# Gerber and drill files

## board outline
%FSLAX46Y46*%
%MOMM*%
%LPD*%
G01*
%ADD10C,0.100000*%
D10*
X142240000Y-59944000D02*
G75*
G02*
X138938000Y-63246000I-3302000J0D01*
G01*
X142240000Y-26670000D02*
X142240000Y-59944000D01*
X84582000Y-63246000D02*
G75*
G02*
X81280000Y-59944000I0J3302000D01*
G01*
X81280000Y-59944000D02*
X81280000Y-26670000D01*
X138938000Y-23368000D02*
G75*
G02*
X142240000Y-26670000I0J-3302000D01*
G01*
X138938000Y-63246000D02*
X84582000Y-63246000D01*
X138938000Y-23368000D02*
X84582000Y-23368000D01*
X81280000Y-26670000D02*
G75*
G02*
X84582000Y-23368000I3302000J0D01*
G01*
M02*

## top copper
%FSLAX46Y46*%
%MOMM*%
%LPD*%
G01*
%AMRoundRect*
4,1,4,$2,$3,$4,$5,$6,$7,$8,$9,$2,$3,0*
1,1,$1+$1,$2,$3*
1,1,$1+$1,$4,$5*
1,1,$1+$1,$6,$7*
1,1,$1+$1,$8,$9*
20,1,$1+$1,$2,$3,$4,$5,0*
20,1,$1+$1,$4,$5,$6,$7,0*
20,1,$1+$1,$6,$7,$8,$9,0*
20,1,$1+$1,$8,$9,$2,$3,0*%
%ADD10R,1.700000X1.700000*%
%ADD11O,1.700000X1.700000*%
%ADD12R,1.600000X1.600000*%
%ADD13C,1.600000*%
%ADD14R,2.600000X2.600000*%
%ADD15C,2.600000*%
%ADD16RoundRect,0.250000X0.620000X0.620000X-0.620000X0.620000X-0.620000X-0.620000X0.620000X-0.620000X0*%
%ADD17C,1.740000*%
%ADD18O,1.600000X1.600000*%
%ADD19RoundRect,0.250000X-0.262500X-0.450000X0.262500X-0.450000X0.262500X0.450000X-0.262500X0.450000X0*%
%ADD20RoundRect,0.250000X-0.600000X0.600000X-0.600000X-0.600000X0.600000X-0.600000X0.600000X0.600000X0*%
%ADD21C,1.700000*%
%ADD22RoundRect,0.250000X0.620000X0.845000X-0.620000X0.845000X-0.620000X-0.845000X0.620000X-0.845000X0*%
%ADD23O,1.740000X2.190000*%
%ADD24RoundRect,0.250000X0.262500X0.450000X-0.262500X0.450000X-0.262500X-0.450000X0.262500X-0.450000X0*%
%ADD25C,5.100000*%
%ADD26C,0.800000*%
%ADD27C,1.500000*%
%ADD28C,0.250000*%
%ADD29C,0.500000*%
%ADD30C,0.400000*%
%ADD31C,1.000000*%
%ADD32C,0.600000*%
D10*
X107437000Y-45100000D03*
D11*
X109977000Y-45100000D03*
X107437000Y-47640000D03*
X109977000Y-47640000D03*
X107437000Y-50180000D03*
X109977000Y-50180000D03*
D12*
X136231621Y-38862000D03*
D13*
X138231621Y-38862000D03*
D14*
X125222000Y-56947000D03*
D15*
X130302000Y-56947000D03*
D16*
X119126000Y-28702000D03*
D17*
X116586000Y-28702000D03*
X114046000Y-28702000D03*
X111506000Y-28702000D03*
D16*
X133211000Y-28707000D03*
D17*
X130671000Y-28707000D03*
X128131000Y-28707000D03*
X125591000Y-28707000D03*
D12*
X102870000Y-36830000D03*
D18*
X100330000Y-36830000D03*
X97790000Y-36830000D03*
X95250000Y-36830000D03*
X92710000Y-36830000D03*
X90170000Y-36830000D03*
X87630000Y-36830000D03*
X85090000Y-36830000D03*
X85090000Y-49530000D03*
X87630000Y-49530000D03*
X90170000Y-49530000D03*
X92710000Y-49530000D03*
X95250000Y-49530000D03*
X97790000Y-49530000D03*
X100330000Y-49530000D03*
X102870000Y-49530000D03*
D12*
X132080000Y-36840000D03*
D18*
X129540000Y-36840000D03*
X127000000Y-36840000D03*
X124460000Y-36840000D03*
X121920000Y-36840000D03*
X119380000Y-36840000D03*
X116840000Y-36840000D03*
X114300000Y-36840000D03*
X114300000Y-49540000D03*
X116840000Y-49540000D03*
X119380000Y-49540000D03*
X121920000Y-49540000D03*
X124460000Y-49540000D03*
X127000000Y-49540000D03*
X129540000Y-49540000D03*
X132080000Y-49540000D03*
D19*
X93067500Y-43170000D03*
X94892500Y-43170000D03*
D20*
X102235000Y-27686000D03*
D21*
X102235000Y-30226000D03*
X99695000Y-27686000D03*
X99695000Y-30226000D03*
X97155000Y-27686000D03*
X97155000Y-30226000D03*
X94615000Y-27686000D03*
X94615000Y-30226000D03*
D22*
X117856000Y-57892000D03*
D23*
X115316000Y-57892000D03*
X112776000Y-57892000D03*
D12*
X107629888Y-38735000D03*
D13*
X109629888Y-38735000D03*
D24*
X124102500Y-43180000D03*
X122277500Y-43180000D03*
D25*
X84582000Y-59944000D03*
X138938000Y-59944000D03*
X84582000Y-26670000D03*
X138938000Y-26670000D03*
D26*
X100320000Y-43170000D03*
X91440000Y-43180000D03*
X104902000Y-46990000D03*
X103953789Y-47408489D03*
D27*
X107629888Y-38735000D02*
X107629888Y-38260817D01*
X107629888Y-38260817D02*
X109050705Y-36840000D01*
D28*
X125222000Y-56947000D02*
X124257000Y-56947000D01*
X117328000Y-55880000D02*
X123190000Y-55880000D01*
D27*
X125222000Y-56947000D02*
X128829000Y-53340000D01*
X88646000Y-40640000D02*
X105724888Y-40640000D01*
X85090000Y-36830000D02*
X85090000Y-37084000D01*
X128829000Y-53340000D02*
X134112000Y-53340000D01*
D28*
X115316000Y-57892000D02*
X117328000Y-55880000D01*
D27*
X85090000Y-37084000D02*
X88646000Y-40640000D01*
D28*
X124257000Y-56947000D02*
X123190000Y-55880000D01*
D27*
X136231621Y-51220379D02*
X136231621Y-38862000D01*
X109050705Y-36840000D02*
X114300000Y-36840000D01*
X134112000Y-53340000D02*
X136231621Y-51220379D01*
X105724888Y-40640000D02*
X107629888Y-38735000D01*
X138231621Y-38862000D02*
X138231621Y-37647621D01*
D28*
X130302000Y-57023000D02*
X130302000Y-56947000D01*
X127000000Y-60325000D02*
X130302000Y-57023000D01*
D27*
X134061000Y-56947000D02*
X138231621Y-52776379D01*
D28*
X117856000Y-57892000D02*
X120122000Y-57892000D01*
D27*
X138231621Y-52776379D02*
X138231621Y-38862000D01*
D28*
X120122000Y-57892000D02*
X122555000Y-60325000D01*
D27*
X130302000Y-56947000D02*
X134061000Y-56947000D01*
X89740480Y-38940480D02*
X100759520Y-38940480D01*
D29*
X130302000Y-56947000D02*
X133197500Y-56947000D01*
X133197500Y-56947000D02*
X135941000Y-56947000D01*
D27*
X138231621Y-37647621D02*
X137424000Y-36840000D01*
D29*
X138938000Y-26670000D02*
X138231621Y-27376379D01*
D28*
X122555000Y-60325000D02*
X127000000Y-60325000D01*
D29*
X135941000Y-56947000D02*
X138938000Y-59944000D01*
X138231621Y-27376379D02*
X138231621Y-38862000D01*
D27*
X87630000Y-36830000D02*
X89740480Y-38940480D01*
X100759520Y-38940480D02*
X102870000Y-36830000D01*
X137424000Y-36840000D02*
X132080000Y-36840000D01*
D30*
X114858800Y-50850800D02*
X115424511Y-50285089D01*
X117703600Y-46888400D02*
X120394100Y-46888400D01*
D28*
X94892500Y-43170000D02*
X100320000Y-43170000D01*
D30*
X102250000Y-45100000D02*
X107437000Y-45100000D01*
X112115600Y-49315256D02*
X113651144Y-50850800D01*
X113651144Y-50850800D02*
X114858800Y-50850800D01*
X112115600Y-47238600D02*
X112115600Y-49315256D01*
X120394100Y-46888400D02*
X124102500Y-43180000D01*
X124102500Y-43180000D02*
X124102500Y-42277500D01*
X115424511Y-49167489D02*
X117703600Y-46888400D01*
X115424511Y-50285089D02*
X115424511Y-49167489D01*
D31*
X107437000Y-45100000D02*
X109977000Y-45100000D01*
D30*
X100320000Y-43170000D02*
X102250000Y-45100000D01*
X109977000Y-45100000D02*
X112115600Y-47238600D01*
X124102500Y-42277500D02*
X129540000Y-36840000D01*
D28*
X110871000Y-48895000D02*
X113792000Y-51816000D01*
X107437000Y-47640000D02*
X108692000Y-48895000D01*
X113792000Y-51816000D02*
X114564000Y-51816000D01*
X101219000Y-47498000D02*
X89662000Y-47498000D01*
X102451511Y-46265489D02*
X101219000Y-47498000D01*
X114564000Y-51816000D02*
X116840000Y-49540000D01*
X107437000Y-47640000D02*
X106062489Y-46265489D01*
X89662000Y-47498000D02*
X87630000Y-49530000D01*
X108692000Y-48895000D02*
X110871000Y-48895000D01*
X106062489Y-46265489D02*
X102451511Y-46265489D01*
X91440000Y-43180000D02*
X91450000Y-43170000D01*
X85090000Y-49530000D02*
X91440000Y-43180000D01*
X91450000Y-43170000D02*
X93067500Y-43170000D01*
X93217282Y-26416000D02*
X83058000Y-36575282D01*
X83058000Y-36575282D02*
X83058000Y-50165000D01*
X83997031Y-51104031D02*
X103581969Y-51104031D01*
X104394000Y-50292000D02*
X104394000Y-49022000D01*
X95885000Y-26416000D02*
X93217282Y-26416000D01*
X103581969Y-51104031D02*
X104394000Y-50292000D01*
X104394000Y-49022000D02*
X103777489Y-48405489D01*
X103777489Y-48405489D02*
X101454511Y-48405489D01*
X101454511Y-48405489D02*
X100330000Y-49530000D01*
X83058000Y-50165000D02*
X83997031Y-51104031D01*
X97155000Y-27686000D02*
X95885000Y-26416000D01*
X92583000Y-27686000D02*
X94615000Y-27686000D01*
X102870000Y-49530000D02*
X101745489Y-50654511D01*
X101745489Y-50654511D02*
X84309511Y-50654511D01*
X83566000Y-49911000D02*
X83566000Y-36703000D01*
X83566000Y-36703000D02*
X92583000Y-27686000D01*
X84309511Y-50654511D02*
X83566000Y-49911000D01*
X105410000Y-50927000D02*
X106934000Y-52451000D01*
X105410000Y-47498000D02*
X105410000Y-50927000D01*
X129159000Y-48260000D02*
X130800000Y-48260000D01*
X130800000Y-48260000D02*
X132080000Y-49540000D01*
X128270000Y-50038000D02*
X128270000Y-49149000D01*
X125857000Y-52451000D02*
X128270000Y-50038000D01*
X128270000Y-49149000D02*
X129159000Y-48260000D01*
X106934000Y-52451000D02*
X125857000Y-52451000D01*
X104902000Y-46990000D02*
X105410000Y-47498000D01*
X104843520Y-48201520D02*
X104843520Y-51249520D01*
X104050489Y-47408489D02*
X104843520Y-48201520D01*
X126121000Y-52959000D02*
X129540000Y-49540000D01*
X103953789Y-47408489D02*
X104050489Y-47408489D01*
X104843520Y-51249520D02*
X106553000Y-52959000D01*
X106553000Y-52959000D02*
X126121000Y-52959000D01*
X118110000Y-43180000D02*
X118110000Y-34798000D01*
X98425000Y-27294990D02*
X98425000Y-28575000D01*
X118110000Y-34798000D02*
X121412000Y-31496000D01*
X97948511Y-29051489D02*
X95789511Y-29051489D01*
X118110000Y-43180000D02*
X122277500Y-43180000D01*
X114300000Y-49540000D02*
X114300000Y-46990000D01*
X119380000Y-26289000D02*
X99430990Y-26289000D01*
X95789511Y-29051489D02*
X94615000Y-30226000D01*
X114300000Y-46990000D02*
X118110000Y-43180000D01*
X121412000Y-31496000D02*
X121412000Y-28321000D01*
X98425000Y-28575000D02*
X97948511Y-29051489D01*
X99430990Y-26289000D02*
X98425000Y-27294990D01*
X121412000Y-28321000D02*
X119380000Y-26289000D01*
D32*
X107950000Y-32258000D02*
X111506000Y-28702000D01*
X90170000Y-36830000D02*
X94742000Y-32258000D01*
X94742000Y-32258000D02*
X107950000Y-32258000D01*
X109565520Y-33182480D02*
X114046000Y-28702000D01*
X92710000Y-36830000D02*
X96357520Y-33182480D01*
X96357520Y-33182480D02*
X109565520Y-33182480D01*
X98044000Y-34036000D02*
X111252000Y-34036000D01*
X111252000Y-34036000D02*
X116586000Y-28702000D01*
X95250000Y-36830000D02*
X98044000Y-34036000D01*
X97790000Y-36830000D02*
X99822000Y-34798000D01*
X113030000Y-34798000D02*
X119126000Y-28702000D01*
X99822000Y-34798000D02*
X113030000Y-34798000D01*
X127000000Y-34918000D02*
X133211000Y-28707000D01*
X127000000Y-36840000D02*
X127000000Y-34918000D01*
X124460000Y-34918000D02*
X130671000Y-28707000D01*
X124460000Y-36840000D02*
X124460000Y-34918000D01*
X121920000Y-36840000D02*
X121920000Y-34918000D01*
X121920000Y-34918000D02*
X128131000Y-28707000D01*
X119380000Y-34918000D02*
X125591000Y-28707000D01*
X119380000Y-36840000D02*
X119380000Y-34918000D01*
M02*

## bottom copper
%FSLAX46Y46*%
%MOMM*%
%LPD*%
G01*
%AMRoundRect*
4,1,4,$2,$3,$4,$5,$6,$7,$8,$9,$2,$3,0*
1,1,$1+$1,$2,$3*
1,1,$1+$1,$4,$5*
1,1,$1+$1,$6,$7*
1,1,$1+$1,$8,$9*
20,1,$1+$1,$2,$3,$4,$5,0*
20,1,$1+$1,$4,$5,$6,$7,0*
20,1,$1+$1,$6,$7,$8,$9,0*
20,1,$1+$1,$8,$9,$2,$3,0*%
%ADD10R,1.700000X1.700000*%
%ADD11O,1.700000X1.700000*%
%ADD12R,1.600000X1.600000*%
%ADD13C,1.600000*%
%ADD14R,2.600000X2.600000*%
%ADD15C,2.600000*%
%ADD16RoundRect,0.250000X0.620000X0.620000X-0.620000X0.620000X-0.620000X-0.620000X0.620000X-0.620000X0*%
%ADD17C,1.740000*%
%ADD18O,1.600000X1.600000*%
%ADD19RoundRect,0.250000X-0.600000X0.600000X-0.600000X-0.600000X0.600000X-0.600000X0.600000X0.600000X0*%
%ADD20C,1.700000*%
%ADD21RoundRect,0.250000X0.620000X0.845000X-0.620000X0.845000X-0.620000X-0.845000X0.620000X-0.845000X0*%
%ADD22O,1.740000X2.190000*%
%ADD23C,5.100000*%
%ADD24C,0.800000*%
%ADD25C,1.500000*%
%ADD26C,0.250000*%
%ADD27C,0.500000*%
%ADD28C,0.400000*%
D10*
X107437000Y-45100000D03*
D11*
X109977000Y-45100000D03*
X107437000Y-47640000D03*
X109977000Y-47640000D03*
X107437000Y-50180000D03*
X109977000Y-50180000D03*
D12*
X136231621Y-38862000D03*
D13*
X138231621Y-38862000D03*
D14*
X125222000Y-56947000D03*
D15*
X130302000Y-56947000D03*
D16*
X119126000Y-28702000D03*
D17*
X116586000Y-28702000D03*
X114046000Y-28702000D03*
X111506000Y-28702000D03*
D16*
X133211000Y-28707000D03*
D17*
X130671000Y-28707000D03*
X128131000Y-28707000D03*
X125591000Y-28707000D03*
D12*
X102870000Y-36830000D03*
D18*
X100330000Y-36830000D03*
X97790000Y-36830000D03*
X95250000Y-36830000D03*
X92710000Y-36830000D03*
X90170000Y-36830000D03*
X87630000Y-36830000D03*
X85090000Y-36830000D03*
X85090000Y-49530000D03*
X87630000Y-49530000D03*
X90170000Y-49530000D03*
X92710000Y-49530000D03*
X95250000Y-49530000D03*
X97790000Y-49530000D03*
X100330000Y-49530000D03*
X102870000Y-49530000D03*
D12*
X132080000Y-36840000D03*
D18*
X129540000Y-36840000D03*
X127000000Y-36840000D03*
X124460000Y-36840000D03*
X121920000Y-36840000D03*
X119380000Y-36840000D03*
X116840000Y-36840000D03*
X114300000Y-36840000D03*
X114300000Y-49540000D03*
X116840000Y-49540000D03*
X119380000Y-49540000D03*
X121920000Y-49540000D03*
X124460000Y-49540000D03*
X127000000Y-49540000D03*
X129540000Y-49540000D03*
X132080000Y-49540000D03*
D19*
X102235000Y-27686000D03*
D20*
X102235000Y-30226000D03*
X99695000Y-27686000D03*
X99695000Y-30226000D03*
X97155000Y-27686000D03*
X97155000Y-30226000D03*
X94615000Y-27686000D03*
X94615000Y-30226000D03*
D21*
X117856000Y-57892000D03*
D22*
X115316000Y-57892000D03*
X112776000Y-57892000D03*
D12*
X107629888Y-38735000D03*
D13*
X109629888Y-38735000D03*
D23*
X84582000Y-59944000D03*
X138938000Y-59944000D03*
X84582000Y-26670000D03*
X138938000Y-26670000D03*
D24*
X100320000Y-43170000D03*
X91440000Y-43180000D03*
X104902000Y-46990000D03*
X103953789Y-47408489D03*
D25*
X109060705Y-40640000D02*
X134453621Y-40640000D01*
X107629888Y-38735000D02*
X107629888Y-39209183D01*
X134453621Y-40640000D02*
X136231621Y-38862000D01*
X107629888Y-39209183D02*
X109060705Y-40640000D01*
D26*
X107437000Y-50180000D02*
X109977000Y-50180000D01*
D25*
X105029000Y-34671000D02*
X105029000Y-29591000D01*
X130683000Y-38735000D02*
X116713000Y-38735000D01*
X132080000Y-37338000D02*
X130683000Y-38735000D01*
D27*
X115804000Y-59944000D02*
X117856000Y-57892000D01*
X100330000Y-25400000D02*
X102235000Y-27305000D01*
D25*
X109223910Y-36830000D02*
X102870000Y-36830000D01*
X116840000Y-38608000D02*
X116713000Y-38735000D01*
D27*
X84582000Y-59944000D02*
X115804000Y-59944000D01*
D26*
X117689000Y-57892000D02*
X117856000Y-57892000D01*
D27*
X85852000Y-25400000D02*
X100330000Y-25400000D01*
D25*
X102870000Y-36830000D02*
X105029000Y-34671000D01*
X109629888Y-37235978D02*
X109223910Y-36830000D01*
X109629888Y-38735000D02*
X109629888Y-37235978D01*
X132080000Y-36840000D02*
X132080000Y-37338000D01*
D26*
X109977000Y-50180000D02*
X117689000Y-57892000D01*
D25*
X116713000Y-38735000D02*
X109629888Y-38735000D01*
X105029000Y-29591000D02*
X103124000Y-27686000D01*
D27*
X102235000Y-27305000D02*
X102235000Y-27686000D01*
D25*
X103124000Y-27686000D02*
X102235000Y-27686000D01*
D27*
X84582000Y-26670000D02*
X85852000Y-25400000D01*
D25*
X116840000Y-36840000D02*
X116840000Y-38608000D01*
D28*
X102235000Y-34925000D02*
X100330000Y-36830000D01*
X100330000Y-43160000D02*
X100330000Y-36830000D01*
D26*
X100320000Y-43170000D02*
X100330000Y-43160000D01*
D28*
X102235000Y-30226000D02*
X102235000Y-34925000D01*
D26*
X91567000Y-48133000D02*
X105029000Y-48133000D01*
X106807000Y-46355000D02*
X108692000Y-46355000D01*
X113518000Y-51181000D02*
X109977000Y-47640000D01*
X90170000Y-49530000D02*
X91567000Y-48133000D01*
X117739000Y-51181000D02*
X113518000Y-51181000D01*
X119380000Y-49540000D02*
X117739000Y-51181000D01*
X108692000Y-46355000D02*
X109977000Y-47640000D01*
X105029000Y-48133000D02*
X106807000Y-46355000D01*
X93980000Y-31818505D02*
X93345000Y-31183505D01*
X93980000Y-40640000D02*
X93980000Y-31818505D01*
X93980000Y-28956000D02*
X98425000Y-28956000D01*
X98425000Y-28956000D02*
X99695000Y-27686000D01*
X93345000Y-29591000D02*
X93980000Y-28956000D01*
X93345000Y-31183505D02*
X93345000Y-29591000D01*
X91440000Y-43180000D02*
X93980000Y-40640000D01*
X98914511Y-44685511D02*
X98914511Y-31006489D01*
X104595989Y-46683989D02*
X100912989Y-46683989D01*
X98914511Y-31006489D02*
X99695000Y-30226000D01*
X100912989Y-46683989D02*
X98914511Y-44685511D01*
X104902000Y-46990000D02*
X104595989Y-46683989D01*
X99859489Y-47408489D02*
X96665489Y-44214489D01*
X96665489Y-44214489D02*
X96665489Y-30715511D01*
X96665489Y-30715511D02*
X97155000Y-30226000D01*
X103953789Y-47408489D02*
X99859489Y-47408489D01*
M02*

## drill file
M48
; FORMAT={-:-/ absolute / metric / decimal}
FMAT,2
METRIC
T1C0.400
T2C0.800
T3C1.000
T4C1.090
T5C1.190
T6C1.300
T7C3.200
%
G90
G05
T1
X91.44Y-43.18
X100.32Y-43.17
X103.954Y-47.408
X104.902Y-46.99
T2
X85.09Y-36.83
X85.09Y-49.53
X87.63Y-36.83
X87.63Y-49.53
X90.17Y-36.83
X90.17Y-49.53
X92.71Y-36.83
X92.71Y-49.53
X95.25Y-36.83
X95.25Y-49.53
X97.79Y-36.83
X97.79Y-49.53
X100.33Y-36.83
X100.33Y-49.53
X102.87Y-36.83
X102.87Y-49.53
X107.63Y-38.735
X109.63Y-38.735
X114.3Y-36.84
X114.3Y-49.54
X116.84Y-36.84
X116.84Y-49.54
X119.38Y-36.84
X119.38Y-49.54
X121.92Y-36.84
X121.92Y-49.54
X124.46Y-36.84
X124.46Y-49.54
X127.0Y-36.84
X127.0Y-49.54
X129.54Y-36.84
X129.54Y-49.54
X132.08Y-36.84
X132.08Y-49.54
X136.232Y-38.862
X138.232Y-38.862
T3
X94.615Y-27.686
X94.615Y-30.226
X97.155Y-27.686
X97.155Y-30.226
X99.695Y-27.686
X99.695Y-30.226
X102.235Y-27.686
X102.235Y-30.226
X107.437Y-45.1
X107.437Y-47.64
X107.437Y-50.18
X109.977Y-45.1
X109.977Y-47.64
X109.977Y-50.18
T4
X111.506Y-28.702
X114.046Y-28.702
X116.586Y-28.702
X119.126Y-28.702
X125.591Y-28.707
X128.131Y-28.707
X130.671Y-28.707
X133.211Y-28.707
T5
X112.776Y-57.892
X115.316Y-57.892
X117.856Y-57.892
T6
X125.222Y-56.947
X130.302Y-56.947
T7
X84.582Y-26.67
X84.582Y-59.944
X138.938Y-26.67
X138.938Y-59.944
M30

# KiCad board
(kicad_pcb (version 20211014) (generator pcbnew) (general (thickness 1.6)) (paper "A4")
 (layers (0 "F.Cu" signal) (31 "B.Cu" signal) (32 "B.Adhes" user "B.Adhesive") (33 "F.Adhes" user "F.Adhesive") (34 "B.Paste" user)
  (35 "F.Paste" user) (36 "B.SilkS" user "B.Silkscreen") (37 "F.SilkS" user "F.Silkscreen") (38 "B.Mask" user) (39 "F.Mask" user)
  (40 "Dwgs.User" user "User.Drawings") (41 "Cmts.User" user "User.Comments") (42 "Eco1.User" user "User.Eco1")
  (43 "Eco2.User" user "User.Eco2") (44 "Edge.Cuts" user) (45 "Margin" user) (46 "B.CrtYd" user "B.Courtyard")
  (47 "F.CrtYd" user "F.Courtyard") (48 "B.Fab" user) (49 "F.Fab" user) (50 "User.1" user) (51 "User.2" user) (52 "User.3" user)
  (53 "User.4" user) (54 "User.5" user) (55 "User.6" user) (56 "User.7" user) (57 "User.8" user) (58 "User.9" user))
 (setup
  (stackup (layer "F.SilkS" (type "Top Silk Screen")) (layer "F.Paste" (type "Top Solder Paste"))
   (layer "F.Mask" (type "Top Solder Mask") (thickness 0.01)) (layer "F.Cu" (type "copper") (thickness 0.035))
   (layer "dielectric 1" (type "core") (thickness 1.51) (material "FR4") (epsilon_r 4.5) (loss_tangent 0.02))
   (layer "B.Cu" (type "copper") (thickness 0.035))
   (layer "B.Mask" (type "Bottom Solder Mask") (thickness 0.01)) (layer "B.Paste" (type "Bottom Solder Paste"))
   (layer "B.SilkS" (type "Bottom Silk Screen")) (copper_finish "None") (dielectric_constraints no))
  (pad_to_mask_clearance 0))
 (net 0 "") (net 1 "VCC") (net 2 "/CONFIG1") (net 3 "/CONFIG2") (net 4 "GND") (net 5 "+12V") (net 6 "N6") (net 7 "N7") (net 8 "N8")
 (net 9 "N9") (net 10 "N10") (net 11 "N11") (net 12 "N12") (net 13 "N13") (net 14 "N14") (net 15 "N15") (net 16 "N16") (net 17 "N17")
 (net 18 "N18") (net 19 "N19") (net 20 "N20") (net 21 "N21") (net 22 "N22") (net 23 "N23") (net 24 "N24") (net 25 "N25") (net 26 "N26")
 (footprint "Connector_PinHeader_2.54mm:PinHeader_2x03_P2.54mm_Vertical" (layer "F.Cu") (at 107.437 45.1)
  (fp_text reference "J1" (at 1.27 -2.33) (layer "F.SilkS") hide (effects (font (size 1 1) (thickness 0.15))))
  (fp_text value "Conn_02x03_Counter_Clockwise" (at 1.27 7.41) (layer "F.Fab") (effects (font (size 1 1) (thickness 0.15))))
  (pad "1" thru_hole rect (at 0 0) (size 1.7 1.7) (drill 1) (layers *.Cu *.Mask) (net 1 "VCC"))
  (pad "2" thru_hole oval (at 2.54 0) (size 1.7 1.7) (drill 1) (layers *.Cu *.Mask) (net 1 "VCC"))
  (pad "3" thru_hole oval (at 0 2.54) (size 1.7 1.7) (drill 1) (layers *.Cu *.Mask) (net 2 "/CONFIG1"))
  (pad "4" thru_hole oval (at 2.54 2.54) (size 1.7 1.7) (drill 1) (layers *.Cu *.Mask) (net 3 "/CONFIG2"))
  (pad "5" thru_hole oval (at 0 5.08) (size 1.7 1.7) (drill 1) (layers *.Cu *.Mask) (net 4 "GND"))
  (pad "6" thru_hole oval (at 2.54 5.08) (size 1.7 1.7) (drill 1) (layers *.Cu *.Mask) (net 4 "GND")))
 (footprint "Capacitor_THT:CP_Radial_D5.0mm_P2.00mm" (layer "F.Cu") (at 136.231621 38.862)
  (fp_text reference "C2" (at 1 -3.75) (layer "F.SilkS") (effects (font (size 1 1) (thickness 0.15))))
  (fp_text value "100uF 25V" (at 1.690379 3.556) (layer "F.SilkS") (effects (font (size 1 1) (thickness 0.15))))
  (pad "1" thru_hole rect (at 0 0) (size 1.6 1.6) (drill 0.8) (layers *.Cu *.Mask) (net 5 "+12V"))
  (pad "2" thru_hole circle (at 2 0) (size 1.6 1.6) (drill 0.8) (layers *.Cu *.Mask) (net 4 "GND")))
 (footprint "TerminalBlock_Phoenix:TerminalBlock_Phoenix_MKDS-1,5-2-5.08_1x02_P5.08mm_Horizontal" (layer "F.Cu") (at 125.222 56.947)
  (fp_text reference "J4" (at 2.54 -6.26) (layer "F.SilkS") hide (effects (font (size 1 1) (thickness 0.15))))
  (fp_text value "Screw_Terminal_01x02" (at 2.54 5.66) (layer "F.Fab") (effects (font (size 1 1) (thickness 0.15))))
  (pad "1" thru_hole rect (at 0 0) (size 2.6 2.6) (drill 1.3) (layers *.Cu *.Mask) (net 5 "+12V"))
  (pad "2" thru_hole circle (at 5.08 0) (size 2.6 2.6) (drill 1.3) (layers *.Cu *.Mask) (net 4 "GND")))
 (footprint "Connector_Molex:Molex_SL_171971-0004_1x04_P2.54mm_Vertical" (layer "F.Cu") (at 119.126 28.702 180)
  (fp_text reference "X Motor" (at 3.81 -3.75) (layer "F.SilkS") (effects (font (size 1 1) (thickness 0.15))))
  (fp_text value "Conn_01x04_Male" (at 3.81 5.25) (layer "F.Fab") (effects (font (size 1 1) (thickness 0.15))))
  (pad "1" thru_hole roundrect (at 0 0 180) (size 1.74 1.74) (drill 1.09) (layers *.Cu *.Mask) (roundrect_rratio 0.1436781609) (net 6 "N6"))
  (pad "2" thru_hole circle (at 2.54 0 180) (size 1.74 1.74) (drill 1.09) (layers *.Cu *.Mask) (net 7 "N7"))
  (pad "3" thru_hole circle (at 5.08 0 180) (size 1.74 1.74) (drill 1.09) (layers *.Cu *.Mask) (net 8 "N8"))
  (pad "4" thru_hole circle (at 7.62 0 180) (size 1.74 1.74) (drill 1.09) (layers *.Cu *.Mask) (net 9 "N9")))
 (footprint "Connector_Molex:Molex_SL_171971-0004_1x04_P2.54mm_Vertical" (layer "F.Cu") (at 133.211 28.707 180)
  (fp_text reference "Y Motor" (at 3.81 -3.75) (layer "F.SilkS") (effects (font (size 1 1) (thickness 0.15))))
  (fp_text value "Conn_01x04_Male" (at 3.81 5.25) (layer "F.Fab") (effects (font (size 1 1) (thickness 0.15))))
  (pad "1" thru_hole roundrect (at 0 0 180) (size 1.74 1.74) (drill 1.09) (layers *.Cu *.Mask) (roundrect_rratio 0.1436781609)
   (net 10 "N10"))
  (pad "2" thru_hole circle (at 2.54 0 180) (size 1.74 1.74) (drill 1.09) (layers *.Cu *.Mask) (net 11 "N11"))
  (pad "3" thru_hole circle (at 5.08 0 180) (size 1.74 1.74) (drill 1.09) (layers *.Cu *.Mask) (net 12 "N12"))
  (pad "4" thru_hole circle (at 7.62 0 180) (size 1.74 1.74) (drill 1.09) (layers *.Cu *.Mask) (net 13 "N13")))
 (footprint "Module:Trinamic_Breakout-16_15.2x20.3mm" (layer "F.Cu") (at 102.87 36.83 -90)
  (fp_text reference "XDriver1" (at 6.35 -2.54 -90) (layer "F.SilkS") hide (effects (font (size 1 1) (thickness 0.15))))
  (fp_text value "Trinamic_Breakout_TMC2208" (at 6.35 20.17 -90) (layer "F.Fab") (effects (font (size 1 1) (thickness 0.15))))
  (pad "1" thru_hole rect (at 0 0 270) (size 1.6 1.6) (drill 0.8) (layers *.Cu *.Mask) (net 4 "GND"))
  (pad "2" thru_hole oval (at 0 2.54 270) (size 1.6 1.6) (drill 0.8) (layers *.Cu *.Mask) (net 1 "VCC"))
  (pad "3" thru_hole oval (at 0 5.08 270) (size 1.6 1.6) (drill 0.8) (layers *.Cu *.Mask) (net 6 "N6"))
  (pad "4" thru_hole oval (at 0 7.62 270) (size 1.6 1.6) (drill 0.8) (layers *.Cu *.Mask) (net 7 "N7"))
  (pad "5" thru_hole oval (at 0 10.16 270) (size 1.6 1.6) (drill 0.8) (layers *.Cu *.Mask) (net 8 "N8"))
  (pad "6" thru_hole oval (at 0 12.7 270) (size 1.6 1.6) (drill 0.8) (layers *.Cu *.Mask) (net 9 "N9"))
  (pad "7" thru_hole oval (at 0 15.24 270) (size 1.6 1.6) (drill 0.8) (layers *.Cu *.Mask) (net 4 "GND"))
  (pad "8" thru_hole oval (at 0 17.78 270) (size 1.6 1.6) (drill 0.8) (layers *.Cu *.Mask) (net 5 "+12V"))
  (pad "9" thru_hole oval (at 12.7 17.78 270) (size 1.6 1.6) (drill 0.8) (layers *.Cu *.Mask) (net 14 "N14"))
  (pad "10" thru_hole oval (at 12.7 15.24 270) (size 1.6 1.6) (drill 0.8) (layers *.Cu *.Mask) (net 2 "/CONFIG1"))
  (pad "11" thru_hole oval (at 12.7 12.7 270) (size 1.6 1.6) (drill 0.8) (layers *.Cu *.Mask) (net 3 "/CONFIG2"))
  (pad "12" thru_hole oval (at 12.7 10.16 270) (size 1.6 1.6) (drill 0.8) (layers *.Cu *.Mask) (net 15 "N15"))
  (pad "13" thru_hole oval (at 12.7 7.62 270) (size 1.6 1.6) (drill 0.8) (layers *.Cu *.Mask) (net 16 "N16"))
  (pad "14" thru_hole oval (at 12.7 5.08 270) (size 1.6 1.6) (drill 0.8) (layers *.Cu *.Mask) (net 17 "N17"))
  (pad "15" thru_hole oval (at 12.7 2.54 270) (size 1.6 1.6) (drill 0.8) (layers *.Cu *.Mask) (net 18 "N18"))
  (pad "16" thru_hole oval (at 12.7 0 270) (size 1.6 1.6) (drill 0.8) (layers *.Cu *.Mask) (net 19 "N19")))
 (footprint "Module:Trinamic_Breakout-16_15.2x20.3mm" (layer "F.Cu") (at 132.08 36.84 -90)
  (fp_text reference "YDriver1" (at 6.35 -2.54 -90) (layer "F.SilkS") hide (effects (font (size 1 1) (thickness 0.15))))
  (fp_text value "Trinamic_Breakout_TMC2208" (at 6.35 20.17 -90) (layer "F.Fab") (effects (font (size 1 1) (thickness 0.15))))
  (pad "1" thru_hole rect (at 0 0 270) (size 1.6 1.6) (drill 0.8) (layers *.Cu *.Mask) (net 4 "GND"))
  (pad "2" thru_hole oval (at 0 2.54 270) (size 1.6 1.6) (drill 0.8) (layers *.Cu *.Mask) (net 1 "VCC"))
  (pad "3" thru_hole oval (at 0 5.08 270) (size 1.6 1.6) (drill 0.8) (layers *.Cu *.Mask) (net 10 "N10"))
  (pad "4" thru_hole oval (at 0 7.62 270) (size 1.6 1.6) (drill 0.8) (layers *.Cu *.Mask) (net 11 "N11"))
  (pad "5" thru_hole oval (at 0 10.16 270) (size 1.6 1.6) (drill 0.8) (layers *.Cu *.Mask) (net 12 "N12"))
  (pad "6" thru_hole oval (at 0 12.7 270) (size 1.6 1.6) (drill 0.8) (layers *.Cu *.Mask) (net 13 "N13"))
  (pad "7" thru_hole oval (at 0 15.24 270) (size 1.6 1.6) (drill 0.8) (layers *.Cu *.Mask) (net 4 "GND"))
  (pad "8" thru_hole oval (at 0 17.78 270) (size 1.6 1.6) (drill 0.8) (layers *.Cu *.Mask) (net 5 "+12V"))
  (pad "9" thru_hole oval (at 12.7 17.78 270) (size 1.6 1.6) (drill 0.8) (layers *.Cu *.Mask) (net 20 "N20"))
  (pad "10" thru_hole oval (at 12.7 15.24 270) (size 1.6 1.6) (drill 0.8) (layers *.Cu *.Mask) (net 2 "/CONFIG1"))
  (pad "11" thru_hole oval (at 12.7 12.7 270) (size 1.6 1.6) (drill 0.8) (layers *.Cu *.Mask) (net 3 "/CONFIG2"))
  (pad "12" thru_hole oval (at 12.7 10.16 270) (size 1.6 1.6) (drill 0.8) (layers *.Cu *.Mask) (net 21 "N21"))
  (pad "13" thru_hole oval (at 12.7 7.62 270) (size 1.6 1.6) (drill 0.8) (layers *.Cu *.Mask) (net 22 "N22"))
  (pad "14" thru_hole oval (at 12.7 5.08 270) (size 1.6 1.6) (drill 0.8) (layers *.Cu *.Mask) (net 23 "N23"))
  (pad "15" thru_hole oval (at 12.7 2.54 270) (size 1.6 1.6) (drill 0.8) (layers *.Cu *.Mask) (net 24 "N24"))
  (pad "16" thru_hole oval (at 12.7 0 270) (size 1.6 1.6) (drill 0.8) (layers *.Cu *.Mask) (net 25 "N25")))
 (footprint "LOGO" (layer "F.Cu") (at 101.981 59.817)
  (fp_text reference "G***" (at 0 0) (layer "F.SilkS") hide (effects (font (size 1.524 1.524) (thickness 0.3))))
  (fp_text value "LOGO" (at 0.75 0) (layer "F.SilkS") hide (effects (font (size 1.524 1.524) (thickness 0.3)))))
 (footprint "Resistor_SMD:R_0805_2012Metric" (layer "F.Cu") (at 93.98 43.17)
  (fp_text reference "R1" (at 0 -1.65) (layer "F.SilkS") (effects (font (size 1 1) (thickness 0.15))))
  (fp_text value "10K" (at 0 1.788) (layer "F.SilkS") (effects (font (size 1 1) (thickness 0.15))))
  (pad "1" smd roundrect (at -0.9125 0) (size 1.025 1.4) (layers "F.Cu" "F.Paste" "F.Mask") (roundrect_rratio 0.243902439) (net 14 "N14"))
  (pad "2" smd roundrect (at 0.9125 0) (size 1.025 1.4) (layers "F.Cu" "F.Paste" "F.Mask") (roundrect_rratio 0.243902439) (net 1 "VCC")))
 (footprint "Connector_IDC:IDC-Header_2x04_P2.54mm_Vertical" (layer "F.Cu") (at 102.235 27.686 -90)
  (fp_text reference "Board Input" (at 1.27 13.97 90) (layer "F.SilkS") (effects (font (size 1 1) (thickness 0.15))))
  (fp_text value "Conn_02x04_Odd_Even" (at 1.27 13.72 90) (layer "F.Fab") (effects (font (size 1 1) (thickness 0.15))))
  (pad "1" thru_hole roundrect (at 0 0 270) (size 1.7 1.7) (drill 1) (layers *.Cu *.Mask) (roundrect_rratio 0.1470588235) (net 4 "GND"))
  (pad "2" thru_hole circle (at 2.54 0 270) (size 1.7 1.7) (drill 1) (layers *.Cu *.Mask) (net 1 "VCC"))
  (pad "3" thru_hole circle (at 0 2.54 270) (size 1.7 1.7) (drill 1) (layers *.Cu *.Mask) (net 14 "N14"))
  (pad "4" thru_hole circle (at 2.54 2.54 270) (size 1.7 1.7) (drill 1) (layers *.Cu *.Mask) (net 25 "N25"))
  (pad "5" thru_hole circle (at 0 5.08 270) (size 1.7 1.7) (drill 1) (layers *.Cu *.Mask) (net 18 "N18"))
  (pad "6" thru_hole circle (at 2.54 5.08 270) (size 1.7 1.7) (drill 1) (layers *.Cu *.Mask) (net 24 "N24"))
  (pad "7" thru_hole circle (at 0 7.62 270) (size 1.7 1.7) (drill 1) (layers *.Cu *.Mask) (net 19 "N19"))
  (pad "8" thru_hole circle (at 2.54 7.62 270) (size 1.7 1.7) (drill 1) (layers *.Cu *.Mask) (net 20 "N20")))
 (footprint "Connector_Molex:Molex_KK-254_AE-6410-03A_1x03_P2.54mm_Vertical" (layer "F.Cu") (at 117.856 57.892 180)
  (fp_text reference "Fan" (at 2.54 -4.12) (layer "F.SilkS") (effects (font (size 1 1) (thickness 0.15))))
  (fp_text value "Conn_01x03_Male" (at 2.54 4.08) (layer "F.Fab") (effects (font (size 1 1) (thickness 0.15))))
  (pad "1" thru_hole roundrect (at 0 0 180) (size 1.74 2.19) (drill 1.19) (layers *.Cu *.Mask) (roundrect_rratio 0.1436781609) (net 4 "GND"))
  (pad "2" thru_hole oval (at 2.54 0 180) (size 1.74 2.19) (drill 1.19) (layers *.Cu *.Mask) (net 5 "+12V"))
  (pad "3" thru_hole oval (at 5.08 0 180) (size 1.74 2.19) (drill 1.19) (layers *.Cu *.Mask) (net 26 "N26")))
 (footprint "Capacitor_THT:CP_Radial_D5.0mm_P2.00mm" (layer "F.Cu") (at 107.629888 38.735)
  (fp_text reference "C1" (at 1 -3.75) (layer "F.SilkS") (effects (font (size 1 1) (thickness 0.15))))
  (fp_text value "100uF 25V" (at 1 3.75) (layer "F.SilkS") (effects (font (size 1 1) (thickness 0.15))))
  (pad "1" thru_hole rect (at 0 0) (size 1.6 1.6) (drill 0.8) (layers *.Cu *.Mask) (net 5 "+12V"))
  (pad "2" thru_hole circle (at 2 0) (size 1.6 1.6) (drill 0.8) (layers *.Cu *.Mask) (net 4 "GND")))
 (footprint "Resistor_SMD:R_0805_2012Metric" (layer "F.Cu") (at 123.19 43.18 180)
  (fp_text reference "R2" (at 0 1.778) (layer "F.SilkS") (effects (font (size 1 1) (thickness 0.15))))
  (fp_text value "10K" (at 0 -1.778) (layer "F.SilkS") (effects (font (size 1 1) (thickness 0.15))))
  (pad "1" smd roundrect (at -0.9125 0 180) (size 1.025 1.4) (layers "F.Cu" "F.Paste" "F.Mask") (roundrect_rratio 0.243902439) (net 1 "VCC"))
  (pad "2" smd roundrect (at 0.9125 0 180) (size 1.025 1.4) (layers "F.Cu" "F.Paste" "F.Mask") (roundrect_rratio 0.243902439) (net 20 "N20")))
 (gr_arc (start 142.24 59.944) (mid 141.272867 62.278867) (end 138.938 63.246) (layer "Edge.Cuts") (width 0.1))
 (gr_line (start 142.24 26.67) (end 142.24 59.944) (layer "Edge.Cuts") (width 0.1))
 (gr_arc (start 84.582 63.246) (mid 82.247133 62.278867) (end 81.28 59.944) (layer "Edge.Cuts") (width 0.1))
 (gr_line (start 81.28 59.944) (end 81.28 26.67) (layer "Edge.Cuts") (width 0.1))
 (gr_arc (start 138.938 23.368) (mid 141.272867 24.335133) (end 142.24 26.67) (layer "Edge.Cuts") (width 0.1))
 (gr_line (start 138.938 63.246) (end 84.582 63.246) (layer "Edge.Cuts") (width 0.1))
 (gr_line (start 138.938 23.368) (end 84.582 23.368) (layer "Edge.Cuts") (width 0.1))
 (gr_arc (start 81.28 26.67) (mid 82.247133 24.335133) (end 84.582 23.368) (layer "Edge.Cuts") (width 0.1))
 (segment (start 107.629888 38.735) (end 107.629888 38.260817) (width 1.5) (layer "F.Cu") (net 5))
 (segment (start 107.629888 38.260817) (end 109.050705 36.84) (width 1.5) (layer "F.Cu") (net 5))
 (segment (start 125.222 56.947) (end 124.257 56.947) (width 0.25) (layer "F.Cu") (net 5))
 (segment (start 117.328 55.88) (end 123.19 55.88) (width 0.25) (layer "F.Cu") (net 5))
 (segment (start 125.222 56.947) (end 128.829 53.34) (width 1.5) (layer "F.Cu") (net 5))
 (segment (start 88.646 40.64) (end 105.724888 40.64) (width 1.5) (layer "F.Cu") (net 5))
 (segment (start 85.09 36.83) (end 85.09 37.084) (width 1.5) (layer "F.Cu") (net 5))
 (segment (start 128.829 53.34) (end 134.112 53.34) (width 1.5) (layer "F.Cu") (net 5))
 (segment (start 115.316 57.892) (end 117.328 55.88) (width 0.25) (layer "F.Cu") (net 5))
 (segment (start 85.09 37.084) (end 88.646 40.64) (width 1.5) (layer "F.Cu") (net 5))
 (segment (start 124.257 56.947) (end 123.19 55.88) (width 0.25) (layer "F.Cu") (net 5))
 (segment (start 136.231621 51.220379) (end 136.231621 38.862) (width 1.5) (layer "F.Cu") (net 5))
 (segment (start 109.050705 36.84) (end 114.3 36.84) (width 1.5) (layer "F.Cu") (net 5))
 (segment (start 134.112 53.34) (end 136.231621 51.220379) (width 1.5) (layer "F.Cu") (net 5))
 (segment (start 105.724888 40.64) (end 107.629888 38.735) (width 1.5) (layer "F.Cu") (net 5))
 (segment (start 109.060705 40.64) (end 134.453621 40.64) (width 1.5) (layer "B.Cu") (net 5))
 (segment (start 107.629888 38.735) (end 107.629888 39.209183) (width 1.5) (layer "B.Cu") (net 5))
 (segment (start 134.453621 40.64) (end 136.231621 38.862) (width 1.5) (layer "B.Cu") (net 5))
 (segment (start 107.629888 39.209183) (end 109.060705 40.64) (width 1.5) (layer "B.Cu") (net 5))
 (segment (start 138.231621 38.862) (end 138.231621 37.647621) (width 1.5) (layer "F.Cu") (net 4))
 (segment (start 130.302 57.023) (end 130.302 56.947) (width 0.25) (layer "F.Cu") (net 4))
 (segment (start 127 60.325) (end 130.302 57.023) (width 0.25) (layer "F.Cu") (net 4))
 (segment (start 134.061 56.947) (end 138.231621 52.776379) (width 1.5) (layer "F.Cu") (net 4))
 (segment (start 117.856 57.892) (end 120.122 57.892) (width 0.25) (layer "F.Cu") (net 4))
 (segment (start 138.231621 52.776379) (end 138.231621 38.862) (width 1.5) (layer "F.Cu") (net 4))
 (segment (start 120.122 57.892) (end 122.555 60.325) (width 0.25) (layer "F.Cu") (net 4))
 (segment (start 130.302 56.947) (end 134.061 56.947) (width 1.5) (layer "F.Cu") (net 4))
 (segment (start 89.74048 38.94048) (end 100.75952 38.94048) (width 1.5) (layer "F.Cu") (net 4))
 (segment (start 130.302 56.947) (end 133.1975 56.947) (width 0.5) (layer "F.Cu") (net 4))
 (segment (start 133.1975 56.947) (end 135.941 56.947) (width 0.5) (layer "F.Cu") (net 4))
 (segment (start 138.231621 37.647621) (end 137.424 36.84) (width 1.5) (layer "F.Cu") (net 4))
 (segment (start 138.938 26.67) (end 138.231621 27.376379) (width 0.5) (layer "F.Cu") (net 4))
 (segment (start 122.555 60.325) (end 127 60.325) (width 0.25) (layer "F.Cu") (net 4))
 (segment (start 135.941 56.947) (end 138.938 59.944) (width 0.5) (layer "F.Cu") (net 4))
 (segment (start 138.231621 27.376379) (end 138.231621 38.862) (width 0.5) (layer "F.Cu") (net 4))
 (segment (start 87.63 36.83) (end 89.74048 38.94048) (width 1.5) (layer "F.Cu") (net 4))
 (segment (start 100.75952 38.94048) (end 102.87 36.83) (width 1.5) (layer "F.Cu") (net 4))
 (segment (start 137.424 36.84) (end 132.08 36.84) (width 1.5) (layer "F.Cu") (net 4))
 (via (at 84.582 59.944) (size 5.1) (drill 3.2) (layers "F.Cu" "B.Cu") (free) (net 4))
 (via (at 138.938 59.944) (size 5.1) (drill 3.2) (layers "F.Cu" "B.Cu") (free) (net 4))
 (via (at 84.582 26.67) (size 5.1) (drill 3.2) (layers "F.Cu" "B.Cu") (free) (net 4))
 (via (at 138.938 26.67) (size 5.1) (drill 3.2) (layers "F.Cu" "B.Cu") (free) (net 4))
 (segment (start 107.437 50.18) (end 109.977 50.18) (width 0.25) (layer "B.Cu") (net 4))
 (segment (start 105.029 34.671) (end 105.029 29.591) (width 1.5) (layer "B.Cu") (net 4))
 (segment (start 130.683 38.735) (end 116.713 38.735) (width 1.5) (layer "B.Cu") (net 4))
 (segment (start 132.08 37.338) (end 130.683 38.735) (width 1.5) (layer "B.Cu") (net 4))
 (segment (start 115.804 59.944) (end 117.856 57.892) (width 0.5) (layer "B.Cu") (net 4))
 (segment (start 100.33 25.4) (end 102.235 27.305) (width 0.5) (layer "B.Cu") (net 4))
 (segment (start 109.22391 36.83) (end 102.87 36.83) (width 1.5) (layer "B.Cu") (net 4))
 (segment (start 116.84 38.608) (end 116.713 38.735) (width 1.5) (layer "B.Cu") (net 4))
 (segment (start 84.582 59.944) (end 115.804 59.944) (width 0.5) (layer "B.Cu") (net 4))
 (segment (start 117.689 57.892) (end 117.856 57.892) (width 0.25) (layer "B.Cu") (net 4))
 (segment (start 85.852 25.4) (end 100.33 25.4) (width 0.5) (layer "B.Cu") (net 4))
 (segment (start 102.87 36.83) (end 105.029 34.671) (width 1.5) (layer "B.Cu") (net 4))
 (segment (start 109.629888 37.235978) (end 109.22391 36.83) (width 1.5) (layer "B.Cu") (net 4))
 (segment (start 109.629888 38.735) (end 109.629888 37.235978) (width 1.5) (layer "B.Cu") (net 4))
 (segment (start 132.08 36.84) (end 132.08 37.338) (width 1.5) (layer "B.Cu") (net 4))
 (segment (start 109.977 50.18) (end 117.689 57.892) (width 0.25) (layer "B.Cu") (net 4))
 (segment (start 116.713 38.735) (end 109.629888 38.735) (width 1.5) (layer "B.Cu") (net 4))
 (segment (start 105.029 29.591) (end 103.124 27.686) (width 1.5) (layer "B.Cu") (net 4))
 (segment (start 102.235 27.305) (end 102.235 27.686) (width 0.5) (layer "B.Cu") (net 4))
 (segment (start 103.124 27.686) (end 102.235 27.686) (width 1.5) (layer "B.Cu") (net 4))
 (segment (start 84.582 26.67) (end 85.852 25.4) (width 0.5) (layer "B.Cu") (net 4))
 (segment (start 116.84 36.84) (end 116.84 38.608) (width 1.5) (layer "B.Cu") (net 4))
 (segment (start 114.8588 50.8508) (end 115.424511 50.285089) (width 0.4) (layer "F.Cu") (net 1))
 (segment (start 117.7036 46.8884) (end 120.3941 46.8884) (width 0.4) (layer "F.Cu") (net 1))
 (segment (start 94.8925 43.17) (end 100.32 43.17) (width 0.25) (layer "F.Cu") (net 1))
 (segment (start 102.25 45.1) (end 107.437 45.1) (width 0.4) (layer "F.Cu") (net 1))
 (segment (start 112.1156 49.315256) (end 113.651144 50.8508) (width 0.4) (layer "F.Cu") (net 1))
 (segment (start 113.651144 50.8508) (end 114.8588 50.8508) (width 0.4) (layer "F.Cu") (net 1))
 (segment (start 112.1156 47.2386) (end 112.1156 49.315256) (width 0.4) (layer "F.Cu") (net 1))
 (segment (start 120.3941 46.8884) (end 124.1025 43.18) (width 0.4) (layer "F.Cu") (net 1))
 (segment (start 124.1025 43.18) (end 124.1025 42.2775) (width 0.4) (layer "F.Cu") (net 1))
 (segment (start 115.424511 49.167489) (end 117.7036 46.8884) (width 0.4) (layer "F.Cu") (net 1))
 (segment (start 115.424511 50.285089) (end 115.424511 49.167489) (width 0.4) (layer "F.Cu") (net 1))
 (segment (start 107.437 45.1) (end 109.977 45.1) (width 1) (layer "F.Cu") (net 1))
 (segment (start 100.32 43.17) (end 102.25 45.1) (width 0.4) (layer "F.Cu") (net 1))
 (segment (start 109.977 45.1) (end 112.1156 47.2386) (width 0.4) (layer "F.Cu") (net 1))
 (segment (start 124.1025 42.2775) (end 129.54 36.84) (width 0.4) (layer "F.Cu") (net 1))
 (via (at 100.32 43.17) (size 0.8) (drill 0.4) (layers "F.Cu" "B.Cu") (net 1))
 (segment (start 102.235 34.925) (end 100.33 36.83) (width 0.4) (layer "B.Cu") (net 1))
 (segment (start 100.33 43.16) (end 100.33 36.83) (width 0.4) (layer "B.Cu") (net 1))
 (segment (start 100.32 43.17) (end 100.33 43.16) (width 0.25) (layer "B.Cu") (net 1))
 (segment (start 102.235 30.226) (end 102.235 34.925) (width 0.4) (layer "B.Cu") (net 1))
 (segment (start 110.871 48.895) (end 113.792 51.816) (width 0.25) (layer "F.Cu") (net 2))
 (segment (start 107.437 47.64) (end 108.692 48.895) (width 0.25) (layer "F.Cu") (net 2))
 (segment (start 113.792 51.816) (end 114.564 51.816) (width 0.25) (layer "F.Cu") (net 2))
 (segment (start 101.219 47.498) (end 89.662 47.498) (width 0.25) (layer "F.Cu") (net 2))
 (segment (start 102.451511 46.265489) (end 101.219 47.498) (width 0.25) (layer "F.Cu") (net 2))
 (segment (start 114.564 51.816) (end 116.84 49.54) (width 0.25) (layer "F.Cu") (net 2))
 (segment (start 107.437 47.64) (end 106.062489 46.265489) (width 0.25) (layer "F.Cu") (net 2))
 (segment (start 89.662 47.498) (end 87.63 49.53) (width 0.25) (layer "F.Cu") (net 2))
 (segment (start 108.692 48.895) (end 110.871 48.895) (width 0.25) (layer "F.Cu") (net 2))
 (segment (start 106.062489 46.265489) (end 102.451511 46.265489) (width 0.25) (layer "F.Cu") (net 2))
 (segment (start 91.567 48.133) (end 105.029 48.133) (width 0.25) (layer "B.Cu") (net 3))
 (segment (start 106.807 46.355) (end 108.692 46.355) (width 0.25) (layer "B.Cu") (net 3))
 (segment (start 113.518 51.181) (end 109.977 47.64) (width 0.25) (layer "B.Cu") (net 3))
 (segment (start 90.17 49.53) (end 91.567 48.133) (width 0.25) (layer "B.Cu") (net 3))
 (segment (start 117.739 51.181) (end 113.518 51.181) (width 0.25) (layer "B.Cu") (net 3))
 (segment (start 119.38 49.54) (end 117.739 51.181) (width 0.25) (layer "B.Cu") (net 3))
 (segment (start 108.692 46.355) (end 109.977 47.64) (width 0.25) (layer "B.Cu") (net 3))
 (segment (start 105.029 48.133) (end 106.807 46.355) (width 0.25) (layer "B.Cu") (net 3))
 (segment (start 91.44 43.18) (end 91.45 43.17) (width 0.25) (layer "F.Cu") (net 14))
 (segment (start 85.09 49.53) (end 91.44 43.18) (width 0.25) (layer "F.Cu") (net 14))
 (segment (start 91.45 43.17) (end 93.0675 43.17) (width 0.25) (layer "F.Cu") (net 14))
 (via (at 91.44 43.18) (size 0.8) (drill 0.4) (layers "F.Cu" "B.Cu") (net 14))
 (segment (start 93.98 31.818505) (end 93.345 31.183505) (width 0.25) (layer "B.Cu") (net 14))
 (segment (start 93.98 40.64) (end 93.98 31.818505) (width 0.25) (layer "B.Cu") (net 14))
 (segment (start 93.98 28.956) (end 98.425 28.956) (width 0.25) (layer "B.Cu") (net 14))
 (segment (start 98.425 28.956) (end 99.695 27.686) (width 0.25) (layer "B.Cu") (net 14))
 (segment (start 93.345 29.591) (end 93.98 28.956) (width 0.25) (layer "B.Cu") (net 14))
 (segment (start 93.345 31.183505) (end 93.345 29.591) (width 0.25) (layer "B.Cu") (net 14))
 (segment (start 91.44 43.18) (end 93.98 40.64) (width 0.25) (layer "B.Cu") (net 14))
 (segment (start 93.217282 26.416) (end 83.058 36.575282) (width 0.25) (layer "F.Cu") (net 18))
 (segment (start 83.058 36.575282) (end 83.058 50.165) (width 0.25) (layer "F.Cu") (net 18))
 (segment (start 83.997031 51.104031) (end 103.581969 51.104031) (width 0.25) (layer "F.Cu") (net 18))
 (segment (start 104.394 50.292) (end 104.394 49.022) (width 0.25) (layer "F.Cu") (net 18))
 (segment (start 95.885 26.416) (end 93.217282 26.416) (width 0.25) (layer "F.Cu") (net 18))
 (segment (start 103.581969 51.104031) (end 104.394 50.292) (width 0.25) (layer "F.Cu") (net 18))
 (segment (start 104.394 49.022) (end 103.777489 48.405489) (width 0.25) (layer "F.Cu") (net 18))
 (segment (start 103.777489 48.405489) (end 101.454511 48.405489) (width 0.25) (layer "F.Cu") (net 18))
 (segment (start 101.454511 48.405489) (end 100.33 49.53) (width 0.25) (layer "F.Cu") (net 18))
 (segment (start 83.058 50.165) (end 83.997031 51.104031) (width 0.25) (layer "F.Cu") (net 18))
 (segment (start 97.155 27.686) (end 95.885 26.416) (width 0.25) (layer "F.Cu") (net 18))
 (segment (start 92.583 27.686) (end 94.615 27.686) (width 0.25) (layer "F.Cu") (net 19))
 (segment (start 102.87 49.53) (end 101.745489 50.654511) (width 0.25) (layer "F.Cu") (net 19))
 (segment (start 101.745489 50.654511) (end 84.309511 50.654511) (width 0.25) (layer "F.Cu") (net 19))
 (segment (start 83.566 49.911) (end 83.566 36.703) (width 0.25) (layer "F.Cu") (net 19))
 (segment (start 83.566 36.703) (end 92.583 27.686) (width 0.25) (layer "F.Cu") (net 19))
 (segment (start 84.309511 50.654511) (end 83.566 49.911) (width 0.25) (layer "F.Cu") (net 19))
 (segment (start 105.41 50.927) (end 106.934 52.451) (width 0.25) (layer "F.Cu") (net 25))
 (segment (start 105.41 47.498) (end 105.41 50.927) (width 0.25) (layer "F.Cu") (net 25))
 (segment (start 129.159 48.26) (end 130.8 48.26) (width 0.25) (layer "F.Cu") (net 25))
 (segment (start 130.8 48.26) (end 132.08 49.54) (width 0.25) (layer "F.Cu") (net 25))
 (segment (start 128.27 50.038) (end 128.27 49.149) (width 0.25) (layer "F.Cu") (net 25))
 (segment (start 125.857 52.451) (end 128.27 50.038) (width 0.25) (layer "F.Cu") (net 25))
 (segment (start 128.27 49.149) (end 129.159 48.26) (width 0.25) (layer "F.Cu") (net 25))
 (segment (start 106.934 52.451) (end 125.857 52.451) (width 0.25) (layer "F.Cu") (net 25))
 (segment (start 104.902 46.99) (end 105.41 47.498) (width 0.25) (layer "F.Cu") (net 25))
 (via (at 104.902 46.99) (size 0.8) (drill 0.4) (layers "F.Cu" "B.Cu") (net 25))
 (segment (start 98.914511 44.685511) (end 98.914511 31.006489) (width 0.25) (layer "B.Cu") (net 25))
 (segment (start 104.595989 46.683989) (end 100.912989 46.683989) (width 0.25) (layer "B.Cu") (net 25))
 (segment (start 98.914511 31.006489) (end 99.695 30.226) (width 0.25) (layer "B.Cu") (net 25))
 (segment (start 100.912989 46.683989) (end 98.914511 44.685511) (width 0.25) (layer "B.Cu") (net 25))
 (segment (start 104.902 46.99) (end 104.595989 46.683989) (width 0.25) (layer "B.Cu") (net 25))
 (segment (start 104.84352 48.20152) (end 104.84352 51.24952) (width 0.25) (layer "F.Cu") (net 24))
 (segment (start 104.050489 47.408489) (end 104.84352 48.20152) (width 0.25) (layer "F.Cu") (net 24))
 (segment (start 126.121 52.959) (end 129.54 49.54) (width 0.25) (layer "F.Cu") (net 24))
 (segment (start 103.953789 47.408489) (end 104.050489 47.408489) (width 0.25) (layer "F.Cu") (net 24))
 (segment (start 104.84352 51.24952) (end 106.553 52.959) (width 0.25) (layer "F.Cu") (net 24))
 (segment (start 106.553 52.959) (end 126.121 52.959) (width 0.25) (layer "F.Cu") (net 24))
 (via (at 103.953789 47.408489) (size 0.8) (drill 0.4) (layers "F.Cu" "B.Cu") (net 24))
 (segment (start 99.859489 47.408489) (end 96.665489 44.214489) (width 0.25) (layer "B.Cu") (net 24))
 (segment (start 96.665489 44.214489) (end 96.665489 30.715511) (width 0.25) (layer "B.Cu") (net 24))
 (segment (start 96.665489 30.715511) (end 97.155 30.226) (width 0.25) (layer "B.Cu") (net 24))
 (segment (start 103.953789 47.408489) (end 99.859489 47.408489) (width 0.25) (layer "B.Cu") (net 24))
 (segment (start 118.11 43.18) (end 118.11 34.798) (width 0.25) (layer "F.Cu") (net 20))
 (segment (start 98.425 27.29499) (end 98.425 28.575) (width 0.25) (layer "F.Cu") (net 20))
 (segment (start 118.11 34.798) (end 121.412 31.496) (width 0.25) (layer "F.Cu") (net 20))
 (segment (start 97.948511 29.051489) (end 95.789511 29.051489) (width 0.25) (layer "F.Cu") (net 20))
 (segment (start 118.11 43.18) (end 122.2775 43.18) (width 0.25) (layer "F.Cu") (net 20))
 (segment (start 114.3 49.54) (end 114.3 46.99) (width 0.25) (layer "F.Cu") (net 20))
 (segment (start 119.38 26.289) (end 99.43099 26.289) (width 0.25) (layer "F.Cu") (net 20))
 (segment (start 95.789511 29.051489) (end 94.615 30.226) (width 0.25) (layer "F.Cu") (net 20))
 (segment (start 114.3 46.99) (end 118.11 43.18) (width 0.25) (layer "F.Cu") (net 20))
 (segment (start 121.412 31.496) (end 121.412 28.321) (width 0.25) (layer "F.Cu") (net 20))
 (segment (start 98.425 28.575) (end 97.948511 29.051489) (width 0.25) (layer "F.Cu") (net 20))
 (segment (start 99.43099 26.289) (end 98.425 27.29499) (width 0.25) (layer "F.Cu") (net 20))
 (segment (start 121.412 28.321) (end 119.38 26.289) (width 0.25) (layer "F.Cu") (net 20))
 (segment (start 107.95 32.258) (end 111.506 28.702) (width 0.6) (layer "F.Cu") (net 9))
 (segment (start 90.17 36.83) (end 94.742 32.258) (width 0.6) (layer "F.Cu") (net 9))
 (segment (start 94.742 32.258) (end 107.95 32.258) (width 0.6) (layer "F.Cu") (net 9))
 (segment (start 109.56552 33.18248) (end 114.046 28.702) (width 0.6) (layer "F.Cu") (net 8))
 (segment (start 92.71 36.83) (end 96.35752 33.18248) (width 0.6) (layer "F.Cu") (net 8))
 (segment (start 96.35752 33.18248) (end 109.56552 33.18248) (width 0.6) (layer "F.Cu") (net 8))
 (segment (start 98.044 34.036) (end 111.252 34.036) (width 0.6) (layer "F.Cu") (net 7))
 (segment (start 111.252 34.036) (end 116.586 28.702) (width 0.6) (layer "F.Cu") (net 7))
 (segment (start 95.25 36.83) (end 98.044 34.036) (width 0.6) (layer "F.Cu") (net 7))
 (segment (start 97.79 36.83) (end 99.822 34.798) (width 0.6) (layer "F.Cu") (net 6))
 (segment (start 113.03 34.798) (end 119.126 28.702) (width 0.6) (layer "F.Cu") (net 6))
 (segment (start 99.822 34.798) (end 113.03 34.798) (width 0.6) (layer "F.Cu") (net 6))
 (segment (start 127 34.918) (end 133.211 28.707) (width 0.6) (layer "F.Cu") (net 10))
 (segment (start 127 36.84) (end 127 34.918) (width 0.6) (layer "F.Cu") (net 10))
 (segment (start 124.46 34.918) (end 130.671 28.707) (width 0.6) (layer "F.Cu") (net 11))
 (segment (start 124.46 36.84) (end 124.46 34.918) (width 0.6) (layer "F.Cu") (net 11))
 (segment (start 121.92 36.84) (end 121.92 34.918) (width 0.6) (layer "F.Cu") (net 12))
 (segment (start 121.92 34.918) (end 128.131 28.707) (width 0.6) (layer "F.Cu") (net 12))
 (segment (start 119.38 34.918) (end 125.591 28.707) (width 0.6) (layer "F.Cu") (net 13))
 (segment (start 119.38 36.84) (end 119.38 34.918) (width 0.6) (layer "F.Cu") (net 13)))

